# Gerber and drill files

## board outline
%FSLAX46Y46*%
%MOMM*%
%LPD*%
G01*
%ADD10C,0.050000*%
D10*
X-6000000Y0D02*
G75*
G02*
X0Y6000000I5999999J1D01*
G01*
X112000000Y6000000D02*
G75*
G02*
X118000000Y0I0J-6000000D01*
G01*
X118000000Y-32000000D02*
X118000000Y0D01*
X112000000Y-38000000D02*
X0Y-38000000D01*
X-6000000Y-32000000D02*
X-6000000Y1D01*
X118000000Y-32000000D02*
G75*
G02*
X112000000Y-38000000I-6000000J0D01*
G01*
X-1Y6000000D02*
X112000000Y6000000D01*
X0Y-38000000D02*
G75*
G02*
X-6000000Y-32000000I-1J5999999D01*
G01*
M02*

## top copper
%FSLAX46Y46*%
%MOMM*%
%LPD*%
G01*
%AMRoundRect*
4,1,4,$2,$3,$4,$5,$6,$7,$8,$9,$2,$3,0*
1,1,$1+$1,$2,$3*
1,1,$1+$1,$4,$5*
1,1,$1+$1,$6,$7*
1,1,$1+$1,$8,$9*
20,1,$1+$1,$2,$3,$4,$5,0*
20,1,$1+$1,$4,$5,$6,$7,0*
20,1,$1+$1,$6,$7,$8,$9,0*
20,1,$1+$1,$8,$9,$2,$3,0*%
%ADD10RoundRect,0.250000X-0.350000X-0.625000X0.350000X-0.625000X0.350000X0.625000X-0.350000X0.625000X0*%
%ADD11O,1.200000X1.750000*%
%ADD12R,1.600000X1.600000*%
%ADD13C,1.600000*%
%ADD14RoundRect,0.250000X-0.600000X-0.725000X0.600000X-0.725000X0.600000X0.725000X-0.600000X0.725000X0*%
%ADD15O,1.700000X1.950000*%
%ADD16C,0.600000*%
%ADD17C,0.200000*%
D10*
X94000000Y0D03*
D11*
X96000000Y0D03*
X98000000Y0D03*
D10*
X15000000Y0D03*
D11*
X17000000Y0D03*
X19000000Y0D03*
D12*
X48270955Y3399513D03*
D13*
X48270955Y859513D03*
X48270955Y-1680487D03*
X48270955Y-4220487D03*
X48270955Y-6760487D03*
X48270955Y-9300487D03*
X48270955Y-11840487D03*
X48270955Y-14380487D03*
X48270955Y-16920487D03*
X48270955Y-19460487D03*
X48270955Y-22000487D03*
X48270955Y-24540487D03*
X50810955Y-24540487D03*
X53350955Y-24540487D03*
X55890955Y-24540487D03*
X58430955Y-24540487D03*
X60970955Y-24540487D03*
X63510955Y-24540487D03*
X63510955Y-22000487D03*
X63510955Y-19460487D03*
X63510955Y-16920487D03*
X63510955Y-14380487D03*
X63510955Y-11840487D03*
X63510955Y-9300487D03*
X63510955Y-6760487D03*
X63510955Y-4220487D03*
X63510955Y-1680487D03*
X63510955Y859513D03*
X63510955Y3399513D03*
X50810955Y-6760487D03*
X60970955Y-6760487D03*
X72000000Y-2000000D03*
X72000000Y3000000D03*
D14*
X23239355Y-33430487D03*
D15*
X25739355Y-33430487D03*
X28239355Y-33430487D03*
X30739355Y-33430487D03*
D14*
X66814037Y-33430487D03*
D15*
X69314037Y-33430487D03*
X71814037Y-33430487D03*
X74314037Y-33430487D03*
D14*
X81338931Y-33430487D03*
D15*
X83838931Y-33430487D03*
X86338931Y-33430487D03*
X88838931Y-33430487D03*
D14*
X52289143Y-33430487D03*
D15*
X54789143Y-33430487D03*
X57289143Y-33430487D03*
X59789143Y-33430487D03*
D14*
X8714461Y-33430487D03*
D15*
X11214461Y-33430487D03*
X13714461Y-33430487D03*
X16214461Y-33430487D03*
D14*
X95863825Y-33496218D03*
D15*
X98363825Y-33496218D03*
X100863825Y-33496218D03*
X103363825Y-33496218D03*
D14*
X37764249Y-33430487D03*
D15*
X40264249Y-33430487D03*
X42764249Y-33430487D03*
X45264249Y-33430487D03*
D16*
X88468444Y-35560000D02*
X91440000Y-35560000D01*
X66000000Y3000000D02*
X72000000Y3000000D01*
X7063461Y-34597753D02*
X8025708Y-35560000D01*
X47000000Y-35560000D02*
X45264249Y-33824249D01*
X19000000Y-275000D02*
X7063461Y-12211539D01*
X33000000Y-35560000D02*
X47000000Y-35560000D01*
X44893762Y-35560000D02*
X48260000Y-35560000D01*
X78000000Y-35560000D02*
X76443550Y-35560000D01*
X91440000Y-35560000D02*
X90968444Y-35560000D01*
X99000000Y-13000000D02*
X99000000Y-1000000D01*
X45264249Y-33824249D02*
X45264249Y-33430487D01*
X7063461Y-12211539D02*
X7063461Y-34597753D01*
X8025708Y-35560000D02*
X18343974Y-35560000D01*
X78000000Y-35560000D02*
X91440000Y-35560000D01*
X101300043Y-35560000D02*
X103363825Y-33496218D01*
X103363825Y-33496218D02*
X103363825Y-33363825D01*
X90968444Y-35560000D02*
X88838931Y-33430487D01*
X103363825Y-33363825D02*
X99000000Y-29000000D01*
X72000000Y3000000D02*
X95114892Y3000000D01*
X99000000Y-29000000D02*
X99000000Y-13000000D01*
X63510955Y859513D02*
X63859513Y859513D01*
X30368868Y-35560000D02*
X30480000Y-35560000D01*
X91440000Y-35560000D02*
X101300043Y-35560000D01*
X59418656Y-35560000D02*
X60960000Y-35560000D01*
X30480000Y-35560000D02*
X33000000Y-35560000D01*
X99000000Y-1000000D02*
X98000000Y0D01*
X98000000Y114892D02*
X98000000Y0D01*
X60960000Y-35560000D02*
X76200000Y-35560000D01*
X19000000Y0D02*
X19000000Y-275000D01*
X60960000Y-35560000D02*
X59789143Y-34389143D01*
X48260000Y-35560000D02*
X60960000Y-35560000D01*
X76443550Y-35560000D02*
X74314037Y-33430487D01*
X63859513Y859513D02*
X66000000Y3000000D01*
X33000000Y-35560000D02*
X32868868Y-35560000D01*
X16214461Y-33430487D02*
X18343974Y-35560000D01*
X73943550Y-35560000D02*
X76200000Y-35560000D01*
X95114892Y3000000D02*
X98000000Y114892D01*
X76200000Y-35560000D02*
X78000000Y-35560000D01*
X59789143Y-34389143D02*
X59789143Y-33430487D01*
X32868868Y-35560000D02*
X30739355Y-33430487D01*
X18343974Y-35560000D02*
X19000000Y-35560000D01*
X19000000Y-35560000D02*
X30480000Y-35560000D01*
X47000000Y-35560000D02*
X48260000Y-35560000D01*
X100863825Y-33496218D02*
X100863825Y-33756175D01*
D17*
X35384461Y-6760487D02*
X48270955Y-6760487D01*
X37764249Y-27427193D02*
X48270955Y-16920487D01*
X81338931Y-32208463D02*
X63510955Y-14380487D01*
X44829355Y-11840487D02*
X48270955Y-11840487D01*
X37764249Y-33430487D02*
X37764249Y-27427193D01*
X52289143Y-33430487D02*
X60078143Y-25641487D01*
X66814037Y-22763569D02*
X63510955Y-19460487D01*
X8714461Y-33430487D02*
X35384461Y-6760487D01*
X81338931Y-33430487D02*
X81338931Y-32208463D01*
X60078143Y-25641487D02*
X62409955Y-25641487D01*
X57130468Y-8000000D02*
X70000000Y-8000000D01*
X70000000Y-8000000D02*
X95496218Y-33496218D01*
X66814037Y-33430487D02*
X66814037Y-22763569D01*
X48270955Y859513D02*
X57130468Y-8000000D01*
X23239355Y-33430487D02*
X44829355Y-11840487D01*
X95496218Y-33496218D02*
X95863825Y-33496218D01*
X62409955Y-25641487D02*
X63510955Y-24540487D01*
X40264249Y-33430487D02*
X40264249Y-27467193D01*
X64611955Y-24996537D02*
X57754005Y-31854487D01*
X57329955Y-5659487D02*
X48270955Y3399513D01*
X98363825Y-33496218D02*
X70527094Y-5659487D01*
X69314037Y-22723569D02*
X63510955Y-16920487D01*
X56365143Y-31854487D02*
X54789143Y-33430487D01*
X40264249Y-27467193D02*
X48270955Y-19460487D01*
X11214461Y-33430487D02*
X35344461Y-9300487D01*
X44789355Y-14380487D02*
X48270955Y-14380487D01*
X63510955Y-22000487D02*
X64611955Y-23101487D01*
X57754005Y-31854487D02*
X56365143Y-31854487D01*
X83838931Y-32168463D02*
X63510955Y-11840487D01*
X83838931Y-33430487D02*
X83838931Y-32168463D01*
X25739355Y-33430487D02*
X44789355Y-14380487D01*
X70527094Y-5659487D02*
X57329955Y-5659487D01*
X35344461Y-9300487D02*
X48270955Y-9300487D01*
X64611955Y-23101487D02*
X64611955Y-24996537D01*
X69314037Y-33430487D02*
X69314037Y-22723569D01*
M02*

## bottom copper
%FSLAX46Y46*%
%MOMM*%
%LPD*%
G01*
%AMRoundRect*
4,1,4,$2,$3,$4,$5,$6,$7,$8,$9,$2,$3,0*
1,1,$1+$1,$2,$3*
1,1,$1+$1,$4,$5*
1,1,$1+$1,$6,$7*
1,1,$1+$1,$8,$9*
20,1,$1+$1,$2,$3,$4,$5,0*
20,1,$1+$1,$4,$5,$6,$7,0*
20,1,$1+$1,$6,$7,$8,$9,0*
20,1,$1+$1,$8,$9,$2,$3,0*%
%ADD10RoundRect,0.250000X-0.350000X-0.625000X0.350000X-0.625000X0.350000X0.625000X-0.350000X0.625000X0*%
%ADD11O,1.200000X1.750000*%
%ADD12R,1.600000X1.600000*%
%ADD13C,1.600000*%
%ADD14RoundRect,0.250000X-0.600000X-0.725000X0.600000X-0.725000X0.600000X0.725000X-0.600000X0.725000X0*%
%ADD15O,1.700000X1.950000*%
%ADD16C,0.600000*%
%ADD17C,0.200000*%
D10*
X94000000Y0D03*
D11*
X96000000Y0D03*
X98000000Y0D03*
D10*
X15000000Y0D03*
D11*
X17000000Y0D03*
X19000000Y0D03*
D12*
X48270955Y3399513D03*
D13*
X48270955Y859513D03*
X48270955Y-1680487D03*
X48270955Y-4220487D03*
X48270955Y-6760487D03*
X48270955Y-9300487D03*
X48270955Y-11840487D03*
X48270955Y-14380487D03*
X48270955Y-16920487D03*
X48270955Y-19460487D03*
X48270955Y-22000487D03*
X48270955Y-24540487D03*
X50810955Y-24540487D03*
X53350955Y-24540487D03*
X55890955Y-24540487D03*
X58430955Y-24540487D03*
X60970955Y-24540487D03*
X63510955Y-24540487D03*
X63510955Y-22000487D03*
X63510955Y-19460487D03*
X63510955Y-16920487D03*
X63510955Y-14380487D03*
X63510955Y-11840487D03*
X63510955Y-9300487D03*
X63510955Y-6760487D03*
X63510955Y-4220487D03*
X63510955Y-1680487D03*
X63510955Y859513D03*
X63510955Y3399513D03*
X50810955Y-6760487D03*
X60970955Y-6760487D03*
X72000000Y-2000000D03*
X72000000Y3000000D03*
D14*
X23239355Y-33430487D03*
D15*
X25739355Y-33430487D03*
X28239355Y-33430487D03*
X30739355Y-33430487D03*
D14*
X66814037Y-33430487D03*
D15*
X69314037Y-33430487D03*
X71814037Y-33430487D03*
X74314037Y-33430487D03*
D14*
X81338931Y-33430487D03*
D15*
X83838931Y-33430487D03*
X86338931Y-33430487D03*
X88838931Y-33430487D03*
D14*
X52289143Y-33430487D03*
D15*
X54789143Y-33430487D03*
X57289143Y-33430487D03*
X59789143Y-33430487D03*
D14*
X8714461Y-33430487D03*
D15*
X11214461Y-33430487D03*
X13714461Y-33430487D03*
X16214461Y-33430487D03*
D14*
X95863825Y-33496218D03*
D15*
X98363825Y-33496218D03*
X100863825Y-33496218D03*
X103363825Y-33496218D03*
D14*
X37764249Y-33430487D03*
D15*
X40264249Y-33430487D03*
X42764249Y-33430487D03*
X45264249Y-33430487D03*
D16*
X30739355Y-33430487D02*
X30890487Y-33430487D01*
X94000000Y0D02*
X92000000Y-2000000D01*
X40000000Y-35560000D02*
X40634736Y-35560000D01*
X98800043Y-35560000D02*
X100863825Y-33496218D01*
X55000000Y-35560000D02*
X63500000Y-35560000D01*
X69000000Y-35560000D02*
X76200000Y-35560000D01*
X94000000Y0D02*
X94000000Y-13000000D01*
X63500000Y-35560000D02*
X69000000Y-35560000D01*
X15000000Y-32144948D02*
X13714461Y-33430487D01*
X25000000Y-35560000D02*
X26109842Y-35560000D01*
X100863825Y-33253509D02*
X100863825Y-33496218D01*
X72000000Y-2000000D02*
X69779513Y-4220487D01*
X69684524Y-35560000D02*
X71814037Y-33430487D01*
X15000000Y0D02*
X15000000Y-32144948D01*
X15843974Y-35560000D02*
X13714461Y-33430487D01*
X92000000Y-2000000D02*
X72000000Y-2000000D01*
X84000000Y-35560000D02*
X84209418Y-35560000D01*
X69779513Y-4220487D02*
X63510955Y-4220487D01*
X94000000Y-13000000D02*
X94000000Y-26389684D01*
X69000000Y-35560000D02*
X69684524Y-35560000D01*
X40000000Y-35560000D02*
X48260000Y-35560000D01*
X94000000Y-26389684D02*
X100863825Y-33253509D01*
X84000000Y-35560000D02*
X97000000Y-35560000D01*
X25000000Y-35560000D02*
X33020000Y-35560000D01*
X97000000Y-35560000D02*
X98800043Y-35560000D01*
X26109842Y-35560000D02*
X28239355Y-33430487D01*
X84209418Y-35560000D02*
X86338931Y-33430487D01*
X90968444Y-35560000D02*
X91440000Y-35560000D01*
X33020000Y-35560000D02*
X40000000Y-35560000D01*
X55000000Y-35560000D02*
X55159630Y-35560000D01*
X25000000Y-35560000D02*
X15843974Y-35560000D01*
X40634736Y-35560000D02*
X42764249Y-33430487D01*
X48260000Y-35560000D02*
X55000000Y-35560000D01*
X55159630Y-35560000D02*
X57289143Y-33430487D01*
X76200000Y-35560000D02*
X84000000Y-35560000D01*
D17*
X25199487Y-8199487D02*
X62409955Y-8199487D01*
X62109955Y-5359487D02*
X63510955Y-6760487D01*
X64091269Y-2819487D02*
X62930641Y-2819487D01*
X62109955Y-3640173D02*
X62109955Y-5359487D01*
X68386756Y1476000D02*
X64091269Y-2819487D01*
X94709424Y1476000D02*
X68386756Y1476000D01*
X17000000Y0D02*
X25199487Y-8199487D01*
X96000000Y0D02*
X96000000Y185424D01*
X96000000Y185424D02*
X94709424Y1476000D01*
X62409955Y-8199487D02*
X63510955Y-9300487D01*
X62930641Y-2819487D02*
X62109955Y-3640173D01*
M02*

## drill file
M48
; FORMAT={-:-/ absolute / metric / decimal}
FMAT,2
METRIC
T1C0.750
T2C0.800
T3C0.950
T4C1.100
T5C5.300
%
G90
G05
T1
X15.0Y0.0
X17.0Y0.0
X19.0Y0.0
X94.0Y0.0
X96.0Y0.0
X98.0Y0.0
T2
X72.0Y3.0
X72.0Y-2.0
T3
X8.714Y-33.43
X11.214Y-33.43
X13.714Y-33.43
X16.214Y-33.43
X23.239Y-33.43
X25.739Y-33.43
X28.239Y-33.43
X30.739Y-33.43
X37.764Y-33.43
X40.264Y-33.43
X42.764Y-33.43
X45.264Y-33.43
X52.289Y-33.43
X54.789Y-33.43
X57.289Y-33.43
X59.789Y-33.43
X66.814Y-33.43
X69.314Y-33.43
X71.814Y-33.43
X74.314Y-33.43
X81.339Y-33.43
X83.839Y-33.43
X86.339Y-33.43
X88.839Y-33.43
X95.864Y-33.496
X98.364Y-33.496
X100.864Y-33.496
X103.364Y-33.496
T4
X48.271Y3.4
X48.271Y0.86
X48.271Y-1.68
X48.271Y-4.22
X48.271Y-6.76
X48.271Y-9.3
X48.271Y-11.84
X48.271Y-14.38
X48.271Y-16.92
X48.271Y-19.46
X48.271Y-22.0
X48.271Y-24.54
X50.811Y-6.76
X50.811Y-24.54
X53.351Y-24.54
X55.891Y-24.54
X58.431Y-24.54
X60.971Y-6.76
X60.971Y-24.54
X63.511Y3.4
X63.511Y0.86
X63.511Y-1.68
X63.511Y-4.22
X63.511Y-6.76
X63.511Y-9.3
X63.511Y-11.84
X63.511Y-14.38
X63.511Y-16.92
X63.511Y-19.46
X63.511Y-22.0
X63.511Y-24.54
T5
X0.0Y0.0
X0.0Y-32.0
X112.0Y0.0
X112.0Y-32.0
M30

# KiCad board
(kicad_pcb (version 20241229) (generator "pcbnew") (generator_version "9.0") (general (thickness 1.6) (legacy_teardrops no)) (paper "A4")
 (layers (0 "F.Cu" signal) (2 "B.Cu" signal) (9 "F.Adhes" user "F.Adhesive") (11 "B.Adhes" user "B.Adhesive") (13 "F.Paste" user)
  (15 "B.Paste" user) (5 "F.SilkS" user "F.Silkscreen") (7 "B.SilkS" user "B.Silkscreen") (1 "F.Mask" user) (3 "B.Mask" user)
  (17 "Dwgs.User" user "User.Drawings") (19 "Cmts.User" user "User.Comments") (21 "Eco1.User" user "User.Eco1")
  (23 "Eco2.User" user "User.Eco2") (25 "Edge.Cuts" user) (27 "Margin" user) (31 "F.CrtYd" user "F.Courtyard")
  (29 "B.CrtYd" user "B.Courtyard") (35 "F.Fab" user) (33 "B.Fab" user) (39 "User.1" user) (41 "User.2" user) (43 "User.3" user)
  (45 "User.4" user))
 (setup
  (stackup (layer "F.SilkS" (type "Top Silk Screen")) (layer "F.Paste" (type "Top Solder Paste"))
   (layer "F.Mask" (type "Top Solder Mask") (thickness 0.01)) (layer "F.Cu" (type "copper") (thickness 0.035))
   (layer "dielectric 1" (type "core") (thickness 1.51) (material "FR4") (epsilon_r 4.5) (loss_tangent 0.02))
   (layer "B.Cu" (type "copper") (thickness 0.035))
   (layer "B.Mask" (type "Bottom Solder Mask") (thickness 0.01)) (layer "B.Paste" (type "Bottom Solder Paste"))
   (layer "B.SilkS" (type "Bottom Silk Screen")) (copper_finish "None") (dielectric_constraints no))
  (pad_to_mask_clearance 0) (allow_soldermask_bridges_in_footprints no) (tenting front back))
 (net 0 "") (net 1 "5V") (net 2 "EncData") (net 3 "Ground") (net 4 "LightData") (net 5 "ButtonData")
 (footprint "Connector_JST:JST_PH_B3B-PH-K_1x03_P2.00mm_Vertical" (layer "F.Cu") (at 94 0)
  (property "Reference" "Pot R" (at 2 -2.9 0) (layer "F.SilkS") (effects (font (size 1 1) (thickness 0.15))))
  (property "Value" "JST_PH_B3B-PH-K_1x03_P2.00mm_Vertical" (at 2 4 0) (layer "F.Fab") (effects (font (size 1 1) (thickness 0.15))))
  (pad "1" thru_hole roundrect (at 0 0) (size 1.2 1.75) (drill 0.75) (layers "*.Cu" "*.Mask") (remove_unused_layers no)
   (roundrect_rratio 0.208333) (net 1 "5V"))
  (pad "2" thru_hole oval (at 2 0) (size 1.2 1.75) (drill 0.75) (layers "*.Cu" "*.Mask") (remove_unused_layers no) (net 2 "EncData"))
  (pad "3" thru_hole oval (at 4 0) (size 1.2 1.75) (drill 0.75) (layers "*.Cu" "*.Mask") (remove_unused_layers no) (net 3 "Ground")))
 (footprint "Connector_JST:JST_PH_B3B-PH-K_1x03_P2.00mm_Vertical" (layer "F.Cu") (at 15 0)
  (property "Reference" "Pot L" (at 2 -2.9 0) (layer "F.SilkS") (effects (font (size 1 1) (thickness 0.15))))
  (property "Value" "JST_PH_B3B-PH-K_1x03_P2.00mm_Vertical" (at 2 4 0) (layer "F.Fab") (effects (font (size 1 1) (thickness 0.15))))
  (pad "1" thru_hole roundrect (at 0 0) (size 1.2 1.75) (drill 0.75) (layers "*.Cu" "*.Mask") (remove_unused_layers no)
   (roundrect_rratio 0.208333) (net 1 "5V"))
  (pad "2" thru_hole oval (at 2 0) (size 1.2 1.75) (drill 0.75) (layers "*.Cu" "*.Mask") (remove_unused_layers no) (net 2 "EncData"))
  (pad "3" thru_hole oval (at 4 0) (size 1.2 1.75) (drill 0.75) (layers "*.Cu" "*.Mask") (remove_unused_layers no) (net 3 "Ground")))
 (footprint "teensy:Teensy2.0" (layer "F.Cu") (at 55.890955 10.570487 -90)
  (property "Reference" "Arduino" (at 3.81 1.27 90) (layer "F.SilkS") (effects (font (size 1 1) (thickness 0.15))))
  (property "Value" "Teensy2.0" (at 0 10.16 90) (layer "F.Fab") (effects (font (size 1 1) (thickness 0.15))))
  (pad "1" thru_hole rect (at -13.97 7.62 270) (size 1.6 1.6) (drill 1.1) (layers "*.Cu" "*.Mask") (remove_unused_layers no)
   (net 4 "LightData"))
  (pad "2" thru_hole circle (at -11.43 7.62 270) (size 1.6 1.6) (drill 1.1) (layers "*.Cu" "*.Mask") (remove_unused_layers no)
   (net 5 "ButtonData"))
  (pad "3" thru_hole circle (at -8.89 7.62 270) (size 1.6 1.6) (drill 1.1) (layers "*.Cu" "*.Mask") (remove_unused_layers no)
   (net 3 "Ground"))
  (pad "4" thru_hole circle (at -6.35 7.62 270) (size 1.6 1.6) (drill 1.1) (layers "*.Cu" "*.Mask") (remove_unused_layers no)
   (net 3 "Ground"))
  (pad "5" thru_hole circle (at -3.81 7.62 270) (size 1.6 1.6) (drill 1.1) (layers "*.Cu" "*.Mask") (remove_unused_layers no)
   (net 5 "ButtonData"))
  (pad "6" thru_hole circle (at -1.27 7.62 270) (size 1.6 1.6) (drill 1.1) (layers "*.Cu" "*.Mask") (remove_unused_layers no)
   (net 4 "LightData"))
  (pad "7" thru_hole circle (at 1.27 7.62 270) (size 1.6 1.6) (drill 1.1) (layers "*.Cu" "*.Mask") (remove_unused_layers no)
   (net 5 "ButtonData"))
  (pad "8" thru_hole circle (at 3.81 7.62 270) (size 1.6 1.6) (drill 1.1) (layers "*.Cu" "*.Mask") (remove_unused_layers no)
   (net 4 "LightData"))
  (pad "9" thru_hole circle (at 6.35 7.62 270) (size 1.6 1.6) (drill 1.1) (layers "*.Cu" "*.Mask") (remove_unused_layers no)
   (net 5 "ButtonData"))
  (pad "10" thru_hole circle (at 8.89 7.62 270) (size 1.6 1.6) (drill 1.1) (layers "*.Cu" "*.Mask") (remove_unused_layers no)
   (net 4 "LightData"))
  (pad "11" thru_hole circle (at 11.43 7.62 270) (size 1.6 1.6) (drill 1.1) (layers "*.Cu" "*.Mask") (remove_unused_layers no))
  (pad "12" thru_hole circle (at 13.97 7.62 270) (size 1.6 1.6) (drill 1.1) (layers "*.Cu" "*.Mask") (remove_unused_layers no))
  (pad "13" thru_hole circle (at 13.97 5.08 270) (size 1.6 1.6) (drill 1.1) (layers "*.Cu" "*.Mask") (remove_unused_layers no))
  (pad "14" thru_hole circle (at 13.97 2.54 270) (size 1.6 1.6) (drill 1.1) (layers "*.Cu" "*.Mask") (remove_unused_layers no))
  (pad "15" thru_hole circle (at 13.97 0 270) (size 1.6 1.6) (drill 1.1) (layers "*.Cu" "*.Mask") (remove_unused_layers no))
  (pad "16" thru_hole circle (at 13.97 -2.54 270) (size 1.6 1.6) (drill 1.1) (layers "*.Cu" "*.Mask") (remove_unused_layers no))
  (pad "17" thru_hole circle (at 13.97 -5.08 270) (size 1.6 1.6) (drill 1.1) (layers "*.Cu" "*.Mask") (remove_unused_layers no))
  (pad "18" thru_hole circle (at 13.97 -7.62 270) (size 1.6 1.6) (drill 1.1) (layers "*.Cu" "*.Mask") (remove_unused_layers no)
   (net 5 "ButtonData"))
  (pad "19" thru_hole circle (at 11.43 -7.62 270) (size 1.6 1.6) (drill 1.1) (layers "*.Cu" "*.Mask") (remove_unused_layers no)
   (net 4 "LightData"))
  (pad "20" thru_hole circle (at 8.89 -7.62 270) (size 1.6 1.6) (drill 1.1) (layers "*.Cu" "*.Mask") (remove_unused_layers no)
   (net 5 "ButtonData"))
  (pad "21" thru_hole circle (at 6.35 -7.62 270) (size 1.6 1.6) (drill 1.1) (layers "*.Cu" "*.Mask") (remove_unused_layers no)
   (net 4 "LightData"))
  (pad "22" thru_hole circle (at 3.81 -7.62 270) (size 1.6 1.6) (drill 1.1) (layers "*.Cu" "*.Mask") (remove_unused_layers no)
   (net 5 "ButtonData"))
  (pad "23" thru_hole circle (at 1.27 -7.62 270) (size 1.6 1.6) (drill 1.1) (layers "*.Cu" "*.Mask") (remove_unused_layers no)
   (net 4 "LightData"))
  (pad "24" thru_hole circle (at -1.27 -7.62 270) (size 1.6 1.6) (drill 1.1) (layers "*.Cu" "*.Mask") (remove_unused_layers no)
   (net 2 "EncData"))
  (pad "25" thru_hole circle (at -3.81 -7.62 270) (size 1.6 1.6) (drill 1.1) (layers "*.Cu" "*.Mask") (remove_unused_layers no)
   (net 2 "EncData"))
  (pad "26" thru_hole circle (at -6.35 -7.62 270) (size 1.6 1.6) (drill 1.1) (layers "*.Cu" "*.Mask") (remove_unused_layers no) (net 1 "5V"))
  (pad "27" thru_hole circle (at -8.89 -7.62 270) (size 1.6 1.6) (drill 1.1) (layers "*.Cu" "*.Mask") (remove_unused_layers no))
  (pad "28" thru_hole circle (at -11.43 -7.62 270) (size 1.6 1.6) (drill 1.1) (layers "*.Cu" "*.Mask") (remove_unused_layers no)
   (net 3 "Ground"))
  (pad "29" thru_hole circle (at -13.97 -7.62 270) (size 1.6 1.6) (drill 1.1) (layers "*.Cu" "*.Mask") (remove_unused_layers no))
  (pad "30" thru_hole circle (at -3.81 5.08 270) (size 1.6 1.6) (drill 1.1) (layers "*.Cu" "*.Mask") (remove_unused_layers no))
  (pad "31" thru_hole circle (at -3.81 -5.08 270) (size 1.6 1.6) (drill 1.1) (layers "*.Cu" "*.Mask") (remove_unused_layers no)))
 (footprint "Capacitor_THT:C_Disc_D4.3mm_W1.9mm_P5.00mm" (layer "F.Cu") (at 72 2 90)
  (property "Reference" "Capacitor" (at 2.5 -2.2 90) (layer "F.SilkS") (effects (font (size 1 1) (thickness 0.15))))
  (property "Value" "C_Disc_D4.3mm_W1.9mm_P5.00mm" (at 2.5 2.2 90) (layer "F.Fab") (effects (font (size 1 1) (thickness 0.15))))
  (pad "1" thru_hole circle (at 0 0 90) (size 1.6 1.6) (drill 0.8) (layers "*.Cu" "*.Mask") (remove_unused_layers no) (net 1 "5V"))
  (pad "2" thru_hole circle (at 5 0 90) (size 1.6 1.6) (drill 0.8) (layers "*.Cu" "*.Mask") (remove_unused_layers no) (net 3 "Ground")))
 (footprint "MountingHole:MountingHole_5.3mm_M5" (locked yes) (layer "F.Cu") (at 0 0)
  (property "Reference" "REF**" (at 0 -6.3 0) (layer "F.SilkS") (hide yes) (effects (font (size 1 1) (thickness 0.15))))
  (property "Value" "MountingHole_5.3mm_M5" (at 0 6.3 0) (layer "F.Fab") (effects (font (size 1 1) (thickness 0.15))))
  (pad "" np_thru_hole circle (at 0 0) (size 5.3 5.3) (drill 5.3) (layers "*.Cu" "*.Mask")))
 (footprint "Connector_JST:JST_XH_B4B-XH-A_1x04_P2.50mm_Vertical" (layer "F.Cu") (at 23.239355 33.430487)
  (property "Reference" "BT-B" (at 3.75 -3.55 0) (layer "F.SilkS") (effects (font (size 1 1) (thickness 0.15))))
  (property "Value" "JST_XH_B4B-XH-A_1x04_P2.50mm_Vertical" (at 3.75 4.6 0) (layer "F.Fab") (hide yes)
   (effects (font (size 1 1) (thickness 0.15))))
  (pad "1" thru_hole roundrect (at 0 0) (size 1.7 1.95) (drill 0.95) (layers "*.Cu" "*.Mask") (remove_unused_layers no)
   (roundrect_rratio 0.147059) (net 5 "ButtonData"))
  (pad "2" thru_hole oval (at 2.5 0) (size 1.7 1.95) (drill 0.95) (layers "*.Cu" "*.Mask") (remove_unused_layers no) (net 4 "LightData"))
  (pad "3" thru_hole oval (at 5 0) (size 1.7 1.95) (drill 0.95) (layers "*.Cu" "*.Mask") (remove_unused_layers no) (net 1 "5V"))
  (pad "4" thru_hole oval (at 7.5 0) (size 1.7 1.95) (drill 0.95) (layers "*.Cu" "*.Mask") (remove_unused_layers no) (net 3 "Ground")))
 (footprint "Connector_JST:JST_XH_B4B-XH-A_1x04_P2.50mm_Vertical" (layer "F.Cu") (at 66.814037 33.430487)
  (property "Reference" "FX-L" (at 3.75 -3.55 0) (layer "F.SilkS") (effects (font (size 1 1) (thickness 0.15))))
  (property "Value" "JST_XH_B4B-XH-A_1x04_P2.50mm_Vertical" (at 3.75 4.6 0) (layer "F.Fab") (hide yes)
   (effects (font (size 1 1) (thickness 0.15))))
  (pad "1" thru_hole roundrect (at 0 0) (size 1.7 1.95) (drill 0.95) (layers "*.Cu" "*.Mask") (remove_unused_layers no)
   (roundrect_rratio 0.147059) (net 5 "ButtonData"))
  (pad "2" thru_hole oval (at 2.5 0) (size 1.7 1.95) (drill 0.95) (layers "*.Cu" "*.Mask") (remove_unused_layers no) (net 4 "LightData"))
  (pad "3" thru_hole oval (at 5 0) (size 1.7 1.95) (drill 0.95) (layers "*.Cu" "*.Mask") (remove_unused_layers no) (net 1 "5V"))
  (pad "4" thru_hole oval (at 7.5 0) (size 1.7 1.95) (drill 0.95) (layers "*.Cu" "*.Mask") (remove_unused_layers no) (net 3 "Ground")))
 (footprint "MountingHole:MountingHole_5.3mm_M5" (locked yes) (layer "F.Cu") (at 112 0)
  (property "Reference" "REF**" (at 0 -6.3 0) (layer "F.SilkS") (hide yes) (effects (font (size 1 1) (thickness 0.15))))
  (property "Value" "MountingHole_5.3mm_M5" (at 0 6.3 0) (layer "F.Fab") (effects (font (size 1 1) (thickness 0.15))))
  (pad "" np_thru_hole circle (at 0 0) (size 5.3 5.3) (drill 5.3) (layers "*.Cu" "*.Mask")))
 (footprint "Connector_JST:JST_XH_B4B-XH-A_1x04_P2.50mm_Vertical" (layer "F.Cu") (at 81.338931 33.430487)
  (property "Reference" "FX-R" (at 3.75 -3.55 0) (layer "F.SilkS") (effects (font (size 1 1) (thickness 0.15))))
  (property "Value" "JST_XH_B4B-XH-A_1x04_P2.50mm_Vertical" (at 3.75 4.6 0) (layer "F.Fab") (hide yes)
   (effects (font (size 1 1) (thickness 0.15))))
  (pad "1" thru_hole roundrect (at 0 0) (size 1.7 1.95) (drill 0.95) (layers "*.Cu" "*.Mask") (remove_unused_layers no)
   (roundrect_rratio 0.147059) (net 5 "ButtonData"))
  (pad "2" thru_hole oval (at 2.5 0) (size 1.7 1.95) (drill 0.95) (layers "*.Cu" "*.Mask") (remove_unused_layers no) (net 4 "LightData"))
  (pad "3" thru_hole oval (at 5 0) (size 1.7 1.95) (drill 0.95) (layers "*.Cu" "*.Mask") (remove_unused_layers no) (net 1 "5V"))
  (pad "4" thru_hole oval (at 7.5 0) (size 1.7 1.95) (drill 0.95) (layers "*.Cu" "*.Mask") (remove_unused_layers no) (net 3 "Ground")))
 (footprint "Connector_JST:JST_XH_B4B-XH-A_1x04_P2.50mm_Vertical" (layer "F.Cu") (at 52.289143 33.430487)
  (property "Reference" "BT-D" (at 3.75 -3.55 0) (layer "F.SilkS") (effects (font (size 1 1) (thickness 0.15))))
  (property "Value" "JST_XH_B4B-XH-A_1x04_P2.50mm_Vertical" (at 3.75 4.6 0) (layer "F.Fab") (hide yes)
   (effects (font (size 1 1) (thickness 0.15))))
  (pad "1" thru_hole roundrect (at 0 0) (size 1.7 1.95) (drill 0.95) (layers "*.Cu" "*.Mask") (remove_unused_layers no)
   (roundrect_rratio 0.147059) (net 5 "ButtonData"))
  (pad "2" thru_hole oval (at 2.5 0) (size 1.7 1.95) (drill 0.95) (layers "*.Cu" "*.Mask") (remove_unused_layers no) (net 4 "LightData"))
  (pad "3" thru_hole oval (at 5 0) (size 1.7 1.95) (drill 0.95) (layers "*.Cu" "*.Mask") (remove_unused_layers no) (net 1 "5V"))
  (pad "4" thru_hole oval (at 7.5 0) (size 1.7 1.95) (drill 0.95) (layers "*.Cu" "*.Mask") (remove_unused_layers no) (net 3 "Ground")))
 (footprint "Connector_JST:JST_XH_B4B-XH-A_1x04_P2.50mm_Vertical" (layer "F.Cu") (at 8.714461 33.430487)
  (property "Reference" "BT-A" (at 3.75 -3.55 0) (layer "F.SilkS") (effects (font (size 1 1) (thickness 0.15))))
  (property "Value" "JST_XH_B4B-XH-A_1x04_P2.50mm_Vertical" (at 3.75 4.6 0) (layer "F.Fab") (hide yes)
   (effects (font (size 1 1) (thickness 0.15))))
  (pad "1" thru_hole roundrect (at 0 0) (size 1.7 1.95) (drill 0.95) (layers "*.Cu" "*.Mask") (remove_unused_layers no)
   (roundrect_rratio 0.147059) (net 5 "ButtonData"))
  (pad "2" thru_hole oval (at 2.5 0) (size 1.7 1.95) (drill 0.95) (layers "*.Cu" "*.Mask") (remove_unused_layers no) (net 4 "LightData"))
  (pad "3" thru_hole oval (at 5 0) (size 1.7 1.95) (drill 0.95) (layers "*.Cu" "*.Mask") (remove_unused_layers no) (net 1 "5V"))
  (pad "4" thru_hole oval (at 7.5 0) (size 1.7 1.95) (drill 0.95) (layers "*.Cu" "*.Mask") (remove_unused_layers no) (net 3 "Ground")))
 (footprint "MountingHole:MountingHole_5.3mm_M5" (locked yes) (layer "F.Cu") (at 0 32)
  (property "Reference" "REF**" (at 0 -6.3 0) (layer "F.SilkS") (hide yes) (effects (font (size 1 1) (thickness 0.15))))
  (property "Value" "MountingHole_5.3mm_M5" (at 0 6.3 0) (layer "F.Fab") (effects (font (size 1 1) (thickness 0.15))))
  (pad "" np_thru_hole circle (at 0 0) (size 5.3 5.3) (drill 5.3) (layers "*.Cu" "*.Mask")))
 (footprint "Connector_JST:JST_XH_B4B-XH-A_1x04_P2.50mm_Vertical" (layer "F.Cu") (at 95.863825 33.496218)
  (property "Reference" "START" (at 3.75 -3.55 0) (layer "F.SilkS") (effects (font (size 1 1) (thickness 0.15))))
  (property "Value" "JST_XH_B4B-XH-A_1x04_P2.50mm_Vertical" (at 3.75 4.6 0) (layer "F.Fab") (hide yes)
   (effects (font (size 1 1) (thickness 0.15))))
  (pad "1" thru_hole roundrect (at 0 0) (size 1.7 1.95) (drill 0.95) (layers "*.Cu" "*.Mask") (remove_unused_layers no)
   (roundrect_rratio 0.147059) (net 5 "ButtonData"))
  (pad "2" thru_hole oval (at 2.5 0) (size 1.7 1.95) (drill 0.95) (layers "*.Cu" "*.Mask") (remove_unused_layers no) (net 4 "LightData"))
  (pad "3" thru_hole oval (at 5 0) (size 1.7 1.95) (drill 0.95) (layers "*.Cu" "*.Mask") (remove_unused_layers no) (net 1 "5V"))
  (pad "4" thru_hole oval (at 7.5 0) (size 1.7 1.95) (drill 0.95) (layers "*.Cu" "*.Mask") (remove_unused_layers no) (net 3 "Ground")))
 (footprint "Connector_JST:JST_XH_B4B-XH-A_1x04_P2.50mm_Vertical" (layer "F.Cu") (at 37.764249 33.430487)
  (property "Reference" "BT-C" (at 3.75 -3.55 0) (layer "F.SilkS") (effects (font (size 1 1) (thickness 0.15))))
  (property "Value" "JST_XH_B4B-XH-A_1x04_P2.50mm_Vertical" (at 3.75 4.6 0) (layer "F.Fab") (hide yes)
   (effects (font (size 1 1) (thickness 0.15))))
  (pad "1" thru_hole roundrect (at 0 0) (size 1.7 1.95) (drill 0.95) (layers "*.Cu" "*.Mask") (remove_unused_layers no)
   (roundrect_rratio 0.147059) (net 5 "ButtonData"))
  (pad "2" thru_hole oval (at 2.5 0) (size 1.7 1.95) (drill 0.95) (layers "*.Cu" "*.Mask") (remove_unused_layers no) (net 4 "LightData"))
  (pad "3" thru_hole oval (at 5 0) (size 1.7 1.95) (drill 0.95) (layers "*.Cu" "*.Mask") (remove_unused_layers no) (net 1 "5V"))
  (pad "4" thru_hole oval (at 7.5 0) (size 1.7 1.95) (drill 0.95) (layers "*.Cu" "*.Mask") (remove_unused_layers no) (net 3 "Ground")))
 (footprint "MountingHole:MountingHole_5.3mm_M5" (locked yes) (layer "F.Cu") (at 112 32)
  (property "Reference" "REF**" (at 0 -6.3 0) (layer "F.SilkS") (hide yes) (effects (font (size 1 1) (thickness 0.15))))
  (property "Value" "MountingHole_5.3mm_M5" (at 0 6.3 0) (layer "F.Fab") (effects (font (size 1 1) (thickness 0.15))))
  (pad "" np_thru_hole circle (at 0 0) (size 5.3 5.3) (drill 5.3) (layers "*.Cu" "*.Mask")))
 (gr_arc (start -6 0) (mid -4.242641 -4.242641) (end 0 -6) (stroke (width 0.05) (type default)) (layer "Edge.Cuts"))
 (gr_arc (start 112 -6) (mid 116.242641 -4.242641) (end 118 0) (stroke (width 0.05) (type default)) (layer "Edge.Cuts"))
 (gr_line (start 118 32) (end 118 0) (stroke (width 0.05) (type default)) (layer "Edge.Cuts"))
 (gr_line (start 112 38) (end 0 38) (stroke (width 0.05) (type default)) (layer "Edge.Cuts"))
 (gr_line (start -6 32) (end -6 -0.000001) (stroke (width 0.05) (type default)) (layer "Edge.Cuts"))
 (gr_arc (start 118 32) (mid 116.242641 36.242641) (end 112 38) (stroke (width 0.05) (type default)) (layer "Edge.Cuts"))
 (gr_line (start -0.000001 -6) (end 112 -6) (stroke (width 0.05) (type default)) (layer "Edge.Cuts"))
 (gr_arc (start 0 38) (mid -4.242641 36.242641) (end -6 32) (stroke (width 0.05) (type default)) (layer "Edge.Cuts"))
 (segment (start 88.468444 35.56) (end 91.44 35.56) (width 0.6) (layer "F.Cu") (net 3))
 (segment (start 66 -3) (end 72 -3) (width 0.6) (layer "F.Cu") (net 3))
 (segment (start 7.063461 34.597753) (end 8.025708 35.56) (width 0.6) (layer "F.Cu") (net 3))
 (segment (start 47 35.56) (end 45.264249 33.824249) (width 0.6) (layer "F.Cu") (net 3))
 (segment (start 19 0.275) (end 7.063461 12.211539) (width 0.6) (layer "F.Cu") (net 3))
 (segment (start 33 35.56) (end 47 35.56) (width 0.6) (layer "F.Cu") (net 3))
 (segment (start 44.893762 35.56) (end 48.26 35.56) (width 0.6) (layer "F.Cu") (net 3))
 (segment (start 78 35.56) (end 76.44355 35.56) (width 0.6) (layer "F.Cu") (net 3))
 (segment (start 91.44 35.56) (end 90.968444 35.56) (width 0.6) (layer "F.Cu") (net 3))
 (segment (start 99 13) (end 99 1) (width 0.6) (layer "F.Cu") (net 3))
 (segment (start 45.264249 33.824249) (end 45.264249 33.430487) (width 0.6) (layer "F.Cu") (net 3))
 (segment (start 7.063461 12.211539) (end 7.063461 34.597753) (width 0.6) (layer "F.Cu") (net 3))
 (segment (start 8.025708 35.56) (end 18.343974 35.56) (width 0.6) (layer "F.Cu") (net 3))
 (segment (start 78 35.56) (end 91.44 35.56) (width 0.6) (layer "F.Cu") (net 3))
 (segment (start 101.300043 35.56) (end 103.363825 33.496218) (width 0.6) (layer "F.Cu") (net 3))
 (segment (start 103.363825 33.496218) (end 103.363825 33.363825) (width 0.6) (layer "F.Cu") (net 3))
 (segment (start 90.968444 35.56) (end 88.838931 33.430487) (width 0.6) (layer "F.Cu") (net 3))
 (segment (start 103.363825 33.363825) (end 99 29) (width 0.6) (layer "F.Cu") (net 3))
 (segment (start 72 -3) (end 95.114892 -3) (width 0.6) (layer "F.Cu") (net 3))
 (segment (start 99 29) (end 99 13) (width 0.6) (layer "F.Cu") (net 3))
 (segment (start 63.510955 -0.859513) (end 63.859513 -0.859513) (width 0.6) (layer "F.Cu") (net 3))
 (segment (start 30.368868 35.56) (end 30.48 35.56) (width 0.6) (layer "F.Cu") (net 3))
 (segment (start 91.44 35.56) (end 101.300043 35.56) (width 0.6) (layer "F.Cu") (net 3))
 (segment (start 59.418656 35.56) (end 60.96 35.56) (width 0.6) (layer "F.Cu") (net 3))
 (segment (start 30.48 35.56) (end 33 35.56) (width 0.6) (layer "F.Cu") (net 3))
 (segment (start 99 1) (end 98 0) (width 0.6) (layer "F.Cu") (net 3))
 (segment (start 98 -0.114892) (end 98 0) (width 0.6) (layer "F.Cu") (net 3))
 (segment (start 60.96 35.56) (end 76.2 35.56) (width 0.6) (layer "F.Cu") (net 3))
 (segment (start 19 0) (end 19 0.275) (width 0.6) (layer "F.Cu") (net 3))
 (segment (start 60.96 35.56) (end 59.789143 34.389143) (width 0.6) (layer "F.Cu") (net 3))
 (segment (start 48.26 35.56) (end 60.96 35.56) (width 0.6) (layer "F.Cu") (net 3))
 (segment (start 76.44355 35.56) (end 74.314037 33.430487) (width 0.6) (layer "F.Cu") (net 3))
 (segment (start 63.859513 -0.859513) (end 66 -3) (width 0.6) (layer "F.Cu") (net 3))
 (segment (start 33 35.56) (end 32.868868 35.56) (width 0.6) (layer "F.Cu") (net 3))
 (segment (start 16.214461 33.430487) (end 18.343974 35.56) (width 0.6) (layer "F.Cu") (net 3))
 (segment (start 73.94355 35.56) (end 76.2 35.56) (width 0.6) (layer "F.Cu") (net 3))
 (segment (start 95.114892 -3) (end 98 -0.114892) (width 0.6) (layer "F.Cu") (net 3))
 (segment (start 76.2 35.56) (end 78 35.56) (width 0.6) (layer "F.Cu") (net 3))
 (segment (start 59.789143 34.389143) (end 59.789143 33.430487) (width 0.6) (layer "F.Cu") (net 3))
 (segment (start 32.868868 35.56) (end 30.739355 33.430487) (width 0.6) (layer "F.Cu") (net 3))
 (segment (start 18.343974 35.56) (end 19 35.56) (width 0.6) (layer "F.Cu") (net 3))
 (segment (start 19 35.56) (end 30.48 35.56) (width 0.6) (layer "F.Cu") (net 3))
 (segment (start 47 35.56) (end 48.26 35.56) (width 0.6) (layer "F.Cu") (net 3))
 (segment (start 30.739355 33.430487) (end 30.890487 33.430487) (width 0.6) (layer "B.Cu") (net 3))
 (segment (start 100.863825 33.496218) (end 100.863825 33.756175) (width 0.6) (layer "F.Cu") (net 1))
 (segment (start 94 0) (end 92 2) (width 0.6) (layer "B.Cu") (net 1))
 (segment (start 40 35.56) (end 40.634736 35.56) (width 0.6) (layer "B.Cu") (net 1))
 (segment (start 98.800043 35.56) (end 100.863825 33.496218) (width 0.6) (layer "B.Cu") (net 1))
 (segment (start 55 35.56) (end 63.5 35.56) (width 0.6) (layer "B.Cu") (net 1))
 (segment (start 69 35.56) (end 76.2 35.56) (width 0.6) (layer "B.Cu") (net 1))
 (segment (start 94 0) (end 94 13) (width 0.6) (layer "B.Cu") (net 1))
 (segment (start 63.5 35.56) (end 69 35.56) (width 0.6) (layer "B.Cu") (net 1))
 (segment (start 15 32.144948) (end 13.714461 33.430487) (width 0.6) (layer "B.Cu") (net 1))
 (segment (start 25 35.56) (end 26.109842 35.56) (width 0.6) (layer "B.Cu") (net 1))
 (segment (start 100.863825 33.253509) (end 100.863825 33.496218) (width 0.6) (layer "B.Cu") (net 1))
 (segment (start 72 2) (end 69.779513 4.220487) (width 0.6) (layer "B.Cu") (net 1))
 (segment (start 69.684524 35.56) (end 71.814037 33.430487) (width 0.6) (layer "B.Cu") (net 1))
 (segment (start 15 0) (end 15 32.144948) (width 0.6) (layer "B.Cu") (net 1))
 (segment (start 15.843974 35.56) (end 13.714461 33.430487) (width 0.6) (layer "B.Cu") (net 1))
 (segment (start 92 2) (end 72 2) (width 0.6) (layer "B.Cu") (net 1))
 (segment (start 84 35.56) (end 84.209418 35.56) (width 0.6) (layer "B.Cu") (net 1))
 (segment (start 69.779513 4.220487) (end 63.510955 4.220487) (width 0.6) (layer "B.Cu") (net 1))
 (segment (start 94 13) (end 94 26.389684) (width 0.6) (layer "B.Cu") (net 1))
 (segment (start 69 35.56) (end 69.684524 35.56) (width 0.6) (layer "B.Cu") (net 1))
 (segment (start 40 35.56) (end 48.26 35.56) (width 0.6) (layer "B.Cu") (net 1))
 (segment (start 94 26.389684) (end 100.863825 33.253509) (width 0.6) (layer "B.Cu") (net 1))
 (segment (start 84 35.56) (end 97 35.56) (width 0.6) (layer "B.Cu") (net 1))
 (segment (start 25 35.56) (end 33.02 35.56) (width 0.6) (layer "B.Cu") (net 1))
 (segment (start 97 35.56) (end 98.800043 35.56) (width 0.6) (layer "B.Cu") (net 1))
 (segment (start 26.109842 35.56) (end 28.239355 33.430487) (width 0.6) (layer "B.Cu") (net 1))
 (segment (start 84.209418 35.56) (end 86.338931 33.430487) (width 0.6) (layer "B.Cu") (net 1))
 (segment (start 90.968444 35.56) (end 91.44 35.56) (width 0.6) (layer "B.Cu") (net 1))
 (segment (start 33.02 35.56) (end 40 35.56) (width 0.6) (layer "B.Cu") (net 1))
 (segment (start 55 35.56) (end 55.15963 35.56) (width 0.6) (layer "B.Cu") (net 1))
 (segment (start 25 35.56) (end 15.843974 35.56) (width 0.6) (layer "B.Cu") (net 1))
 (segment (start 40.634736 35.56) (end 42.764249 33.430487) (width 0.6) (layer "B.Cu") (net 1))
 (segment (start 48.26 35.56) (end 55 35.56) (width 0.6) (layer "B.Cu") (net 1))
 (segment (start 55.15963 35.56) (end 57.289143 33.430487) (width 0.6) (layer "B.Cu") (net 1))
 (segment (start 76.2 35.56) (end 84 35.56) (width 0.6) (layer "B.Cu") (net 1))
 (segment (start 35.384461 6.760487) (end 48.270955 6.760487) (width 0.2) (layer "F.Cu") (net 5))
 (segment (start 37.764249 27.427193) (end 48.270955 16.920487) (width 0.2) (layer "F.Cu") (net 5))
 (segment (start 81.338931 32.208463) (end 63.510955 14.380487) (width 0.2) (layer "F.Cu") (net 5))
 (segment (start 44.829355 11.840487) (end 48.270955 11.840487) (width 0.2) (layer "F.Cu") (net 5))
 (segment (start 37.764249 33.430487) (end 37.764249 27.427193) (width 0.2) (layer "F.Cu") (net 5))
 (segment (start 52.289143 33.430487) (end 60.078143 25.641487) (width 0.2) (layer "F.Cu") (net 5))
 (segment (start 66.814037 22.763569) (end 63.510955 19.460487) (width 0.2) (layer "F.Cu") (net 5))
 (segment (start 8.714461 33.430487) (end 35.384461 6.760487) (width 0.2) (layer "F.Cu") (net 5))
 (segment (start 81.338931 33.430487) (end 81.338931 32.208463) (width 0.2) (layer "F.Cu") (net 5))
 (segment (start 60.078143 25.641487) (end 62.409955 25.641487) (width 0.2) (layer "F.Cu") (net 5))
 (segment (start 57.130468 8) (end 70 8) (width 0.2) (layer "F.Cu") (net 5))
 (segment (start 70 8) (end 95.496218 33.496218) (width 0.2) (layer "F.Cu") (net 5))
 (segment (start 66.814037 33.430487) (end 66.814037 22.763569) (width 0.2) (layer "F.Cu") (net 5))
 (segment (start 48.270955 -0.859513) (end 57.130468 8) (width 0.2) (layer "F.Cu") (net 5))
 (segment (start 23.239355 33.430487) (end 44.829355 11.840487) (width 0.2) (layer "F.Cu") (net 5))
 (segment (start 95.496218 33.496218) (end 95.863825 33.496218) (width 0.2) (layer "F.Cu") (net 5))
 (segment (start 62.409955 25.641487) (end 63.510955 24.540487) (width 0.2) (layer "F.Cu") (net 5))
 (segment (start 40.264249 33.430487) (end 40.264249 27.467193) (width 0.2) (layer "F.Cu") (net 4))
 (segment (start 64.611955 24.996537) (end 57.754005 31.854487) (width 0.2) (layer "F.Cu") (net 4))
 (segment (start 57.329955 5.659487) (end 48.270955 -3.399513) (width 0.2) (layer "F.Cu") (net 4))
 (segment (start 98.363825 33.496218) (end 70.527094 5.659487) (width 0.2) (layer "F.Cu") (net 4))
 (segment (start 69.314037 22.723569) (end 63.510955 16.920487) (width 0.2) (layer "F.Cu") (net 4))
 (segment (start 56.365143 31.854487) (end 54.789143 33.430487) (width 0.2) (layer "F.Cu") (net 4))
 (segment (start 40.264249 27.467193) (end 48.270955 19.460487) (width 0.2) (layer "F.Cu") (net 4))
 (segment (start 11.214461 33.430487) (end 35.344461 9.300487) (width 0.2) (layer "F.Cu") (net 4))
 (segment (start 44.789355 14.380487) (end 48.270955 14.380487) (width 0.2) (layer "F.Cu") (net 4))
 (segment (start 63.510955 22.000487) (end 64.611955 23.101487) (width 0.2) (layer "F.Cu") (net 4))
 (segment (start 57.754005 31.854487) (end 56.365143 31.854487) (width 0.2) (layer "F.Cu") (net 4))
 (segment (start 83.838931 32.168463) (end 63.510955 11.840487) (width 0.2) (layer "F.Cu") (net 4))
 (segment (start 83.838931 33.430487) (end 83.838931 32.168463) (width 0.2) (layer "F.Cu") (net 4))
 (segment (start 25.739355 33.430487) (end 44.789355 14.380487) (width 0.2) (layer "F.Cu") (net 4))
 (segment (start 70.527094 5.659487) (end 57.329955 5.659487) (width 0.2) (layer "F.Cu") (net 4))
 (segment (start 35.344461 9.300487) (end 48.270955 9.300487) (width 0.2) (layer "F.Cu") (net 4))
 (segment (start 64.611955 23.101487) (end 64.611955 24.996537) (width 0.2) (layer "F.Cu") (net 4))
 (segment (start 69.314037 33.430487) (end 69.314037 22.723569) (width 0.2) (layer "F.Cu") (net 4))
 (segment (start 25.199487 8.199487) (end 62.409955 8.199487) (width 0.2) (layer "B.Cu") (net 2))
 (segment (start 62.109955 5.359487) (end 63.510955 6.760487) (width 0.2) (layer "B.Cu") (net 2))
 (segment (start 64.091269 2.819487) (end 62.930641 2.819487) (width 0.2) (layer "B.Cu") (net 2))
 (segment (start 62.109955 3.640173) (end 62.109955 5.359487) (width 0.2) (layer "B.Cu") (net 2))
 (segment (start 68.386756 -1.476) (end 64.091269 2.819487) (width 0.2) (layer "B.Cu") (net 2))
 (segment (start 94.709424 -1.476) (end 68.386756 -1.476) (width 0.2) (layer "B.Cu") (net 2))
 (segment (start 17 0) (end 25.199487 8.199487) (width 0.2) (layer "B.Cu") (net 2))
 (segment (start 96 0) (end 96 -0.185424) (width 0.2) (layer "B.Cu") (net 2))
 (segment (start 96 -0.185424) (end 94.709424 -1.476) (width 0.2) (layer "B.Cu") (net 2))
 (segment (start 62.409955 8.199487) (end 63.510955 9.300487) (width 0.2) (layer "B.Cu") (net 2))
 (segment (start 62.930641 2.819487) (end 62.109955 3.640173) (width 0.2) (layer "B.Cu") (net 2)))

